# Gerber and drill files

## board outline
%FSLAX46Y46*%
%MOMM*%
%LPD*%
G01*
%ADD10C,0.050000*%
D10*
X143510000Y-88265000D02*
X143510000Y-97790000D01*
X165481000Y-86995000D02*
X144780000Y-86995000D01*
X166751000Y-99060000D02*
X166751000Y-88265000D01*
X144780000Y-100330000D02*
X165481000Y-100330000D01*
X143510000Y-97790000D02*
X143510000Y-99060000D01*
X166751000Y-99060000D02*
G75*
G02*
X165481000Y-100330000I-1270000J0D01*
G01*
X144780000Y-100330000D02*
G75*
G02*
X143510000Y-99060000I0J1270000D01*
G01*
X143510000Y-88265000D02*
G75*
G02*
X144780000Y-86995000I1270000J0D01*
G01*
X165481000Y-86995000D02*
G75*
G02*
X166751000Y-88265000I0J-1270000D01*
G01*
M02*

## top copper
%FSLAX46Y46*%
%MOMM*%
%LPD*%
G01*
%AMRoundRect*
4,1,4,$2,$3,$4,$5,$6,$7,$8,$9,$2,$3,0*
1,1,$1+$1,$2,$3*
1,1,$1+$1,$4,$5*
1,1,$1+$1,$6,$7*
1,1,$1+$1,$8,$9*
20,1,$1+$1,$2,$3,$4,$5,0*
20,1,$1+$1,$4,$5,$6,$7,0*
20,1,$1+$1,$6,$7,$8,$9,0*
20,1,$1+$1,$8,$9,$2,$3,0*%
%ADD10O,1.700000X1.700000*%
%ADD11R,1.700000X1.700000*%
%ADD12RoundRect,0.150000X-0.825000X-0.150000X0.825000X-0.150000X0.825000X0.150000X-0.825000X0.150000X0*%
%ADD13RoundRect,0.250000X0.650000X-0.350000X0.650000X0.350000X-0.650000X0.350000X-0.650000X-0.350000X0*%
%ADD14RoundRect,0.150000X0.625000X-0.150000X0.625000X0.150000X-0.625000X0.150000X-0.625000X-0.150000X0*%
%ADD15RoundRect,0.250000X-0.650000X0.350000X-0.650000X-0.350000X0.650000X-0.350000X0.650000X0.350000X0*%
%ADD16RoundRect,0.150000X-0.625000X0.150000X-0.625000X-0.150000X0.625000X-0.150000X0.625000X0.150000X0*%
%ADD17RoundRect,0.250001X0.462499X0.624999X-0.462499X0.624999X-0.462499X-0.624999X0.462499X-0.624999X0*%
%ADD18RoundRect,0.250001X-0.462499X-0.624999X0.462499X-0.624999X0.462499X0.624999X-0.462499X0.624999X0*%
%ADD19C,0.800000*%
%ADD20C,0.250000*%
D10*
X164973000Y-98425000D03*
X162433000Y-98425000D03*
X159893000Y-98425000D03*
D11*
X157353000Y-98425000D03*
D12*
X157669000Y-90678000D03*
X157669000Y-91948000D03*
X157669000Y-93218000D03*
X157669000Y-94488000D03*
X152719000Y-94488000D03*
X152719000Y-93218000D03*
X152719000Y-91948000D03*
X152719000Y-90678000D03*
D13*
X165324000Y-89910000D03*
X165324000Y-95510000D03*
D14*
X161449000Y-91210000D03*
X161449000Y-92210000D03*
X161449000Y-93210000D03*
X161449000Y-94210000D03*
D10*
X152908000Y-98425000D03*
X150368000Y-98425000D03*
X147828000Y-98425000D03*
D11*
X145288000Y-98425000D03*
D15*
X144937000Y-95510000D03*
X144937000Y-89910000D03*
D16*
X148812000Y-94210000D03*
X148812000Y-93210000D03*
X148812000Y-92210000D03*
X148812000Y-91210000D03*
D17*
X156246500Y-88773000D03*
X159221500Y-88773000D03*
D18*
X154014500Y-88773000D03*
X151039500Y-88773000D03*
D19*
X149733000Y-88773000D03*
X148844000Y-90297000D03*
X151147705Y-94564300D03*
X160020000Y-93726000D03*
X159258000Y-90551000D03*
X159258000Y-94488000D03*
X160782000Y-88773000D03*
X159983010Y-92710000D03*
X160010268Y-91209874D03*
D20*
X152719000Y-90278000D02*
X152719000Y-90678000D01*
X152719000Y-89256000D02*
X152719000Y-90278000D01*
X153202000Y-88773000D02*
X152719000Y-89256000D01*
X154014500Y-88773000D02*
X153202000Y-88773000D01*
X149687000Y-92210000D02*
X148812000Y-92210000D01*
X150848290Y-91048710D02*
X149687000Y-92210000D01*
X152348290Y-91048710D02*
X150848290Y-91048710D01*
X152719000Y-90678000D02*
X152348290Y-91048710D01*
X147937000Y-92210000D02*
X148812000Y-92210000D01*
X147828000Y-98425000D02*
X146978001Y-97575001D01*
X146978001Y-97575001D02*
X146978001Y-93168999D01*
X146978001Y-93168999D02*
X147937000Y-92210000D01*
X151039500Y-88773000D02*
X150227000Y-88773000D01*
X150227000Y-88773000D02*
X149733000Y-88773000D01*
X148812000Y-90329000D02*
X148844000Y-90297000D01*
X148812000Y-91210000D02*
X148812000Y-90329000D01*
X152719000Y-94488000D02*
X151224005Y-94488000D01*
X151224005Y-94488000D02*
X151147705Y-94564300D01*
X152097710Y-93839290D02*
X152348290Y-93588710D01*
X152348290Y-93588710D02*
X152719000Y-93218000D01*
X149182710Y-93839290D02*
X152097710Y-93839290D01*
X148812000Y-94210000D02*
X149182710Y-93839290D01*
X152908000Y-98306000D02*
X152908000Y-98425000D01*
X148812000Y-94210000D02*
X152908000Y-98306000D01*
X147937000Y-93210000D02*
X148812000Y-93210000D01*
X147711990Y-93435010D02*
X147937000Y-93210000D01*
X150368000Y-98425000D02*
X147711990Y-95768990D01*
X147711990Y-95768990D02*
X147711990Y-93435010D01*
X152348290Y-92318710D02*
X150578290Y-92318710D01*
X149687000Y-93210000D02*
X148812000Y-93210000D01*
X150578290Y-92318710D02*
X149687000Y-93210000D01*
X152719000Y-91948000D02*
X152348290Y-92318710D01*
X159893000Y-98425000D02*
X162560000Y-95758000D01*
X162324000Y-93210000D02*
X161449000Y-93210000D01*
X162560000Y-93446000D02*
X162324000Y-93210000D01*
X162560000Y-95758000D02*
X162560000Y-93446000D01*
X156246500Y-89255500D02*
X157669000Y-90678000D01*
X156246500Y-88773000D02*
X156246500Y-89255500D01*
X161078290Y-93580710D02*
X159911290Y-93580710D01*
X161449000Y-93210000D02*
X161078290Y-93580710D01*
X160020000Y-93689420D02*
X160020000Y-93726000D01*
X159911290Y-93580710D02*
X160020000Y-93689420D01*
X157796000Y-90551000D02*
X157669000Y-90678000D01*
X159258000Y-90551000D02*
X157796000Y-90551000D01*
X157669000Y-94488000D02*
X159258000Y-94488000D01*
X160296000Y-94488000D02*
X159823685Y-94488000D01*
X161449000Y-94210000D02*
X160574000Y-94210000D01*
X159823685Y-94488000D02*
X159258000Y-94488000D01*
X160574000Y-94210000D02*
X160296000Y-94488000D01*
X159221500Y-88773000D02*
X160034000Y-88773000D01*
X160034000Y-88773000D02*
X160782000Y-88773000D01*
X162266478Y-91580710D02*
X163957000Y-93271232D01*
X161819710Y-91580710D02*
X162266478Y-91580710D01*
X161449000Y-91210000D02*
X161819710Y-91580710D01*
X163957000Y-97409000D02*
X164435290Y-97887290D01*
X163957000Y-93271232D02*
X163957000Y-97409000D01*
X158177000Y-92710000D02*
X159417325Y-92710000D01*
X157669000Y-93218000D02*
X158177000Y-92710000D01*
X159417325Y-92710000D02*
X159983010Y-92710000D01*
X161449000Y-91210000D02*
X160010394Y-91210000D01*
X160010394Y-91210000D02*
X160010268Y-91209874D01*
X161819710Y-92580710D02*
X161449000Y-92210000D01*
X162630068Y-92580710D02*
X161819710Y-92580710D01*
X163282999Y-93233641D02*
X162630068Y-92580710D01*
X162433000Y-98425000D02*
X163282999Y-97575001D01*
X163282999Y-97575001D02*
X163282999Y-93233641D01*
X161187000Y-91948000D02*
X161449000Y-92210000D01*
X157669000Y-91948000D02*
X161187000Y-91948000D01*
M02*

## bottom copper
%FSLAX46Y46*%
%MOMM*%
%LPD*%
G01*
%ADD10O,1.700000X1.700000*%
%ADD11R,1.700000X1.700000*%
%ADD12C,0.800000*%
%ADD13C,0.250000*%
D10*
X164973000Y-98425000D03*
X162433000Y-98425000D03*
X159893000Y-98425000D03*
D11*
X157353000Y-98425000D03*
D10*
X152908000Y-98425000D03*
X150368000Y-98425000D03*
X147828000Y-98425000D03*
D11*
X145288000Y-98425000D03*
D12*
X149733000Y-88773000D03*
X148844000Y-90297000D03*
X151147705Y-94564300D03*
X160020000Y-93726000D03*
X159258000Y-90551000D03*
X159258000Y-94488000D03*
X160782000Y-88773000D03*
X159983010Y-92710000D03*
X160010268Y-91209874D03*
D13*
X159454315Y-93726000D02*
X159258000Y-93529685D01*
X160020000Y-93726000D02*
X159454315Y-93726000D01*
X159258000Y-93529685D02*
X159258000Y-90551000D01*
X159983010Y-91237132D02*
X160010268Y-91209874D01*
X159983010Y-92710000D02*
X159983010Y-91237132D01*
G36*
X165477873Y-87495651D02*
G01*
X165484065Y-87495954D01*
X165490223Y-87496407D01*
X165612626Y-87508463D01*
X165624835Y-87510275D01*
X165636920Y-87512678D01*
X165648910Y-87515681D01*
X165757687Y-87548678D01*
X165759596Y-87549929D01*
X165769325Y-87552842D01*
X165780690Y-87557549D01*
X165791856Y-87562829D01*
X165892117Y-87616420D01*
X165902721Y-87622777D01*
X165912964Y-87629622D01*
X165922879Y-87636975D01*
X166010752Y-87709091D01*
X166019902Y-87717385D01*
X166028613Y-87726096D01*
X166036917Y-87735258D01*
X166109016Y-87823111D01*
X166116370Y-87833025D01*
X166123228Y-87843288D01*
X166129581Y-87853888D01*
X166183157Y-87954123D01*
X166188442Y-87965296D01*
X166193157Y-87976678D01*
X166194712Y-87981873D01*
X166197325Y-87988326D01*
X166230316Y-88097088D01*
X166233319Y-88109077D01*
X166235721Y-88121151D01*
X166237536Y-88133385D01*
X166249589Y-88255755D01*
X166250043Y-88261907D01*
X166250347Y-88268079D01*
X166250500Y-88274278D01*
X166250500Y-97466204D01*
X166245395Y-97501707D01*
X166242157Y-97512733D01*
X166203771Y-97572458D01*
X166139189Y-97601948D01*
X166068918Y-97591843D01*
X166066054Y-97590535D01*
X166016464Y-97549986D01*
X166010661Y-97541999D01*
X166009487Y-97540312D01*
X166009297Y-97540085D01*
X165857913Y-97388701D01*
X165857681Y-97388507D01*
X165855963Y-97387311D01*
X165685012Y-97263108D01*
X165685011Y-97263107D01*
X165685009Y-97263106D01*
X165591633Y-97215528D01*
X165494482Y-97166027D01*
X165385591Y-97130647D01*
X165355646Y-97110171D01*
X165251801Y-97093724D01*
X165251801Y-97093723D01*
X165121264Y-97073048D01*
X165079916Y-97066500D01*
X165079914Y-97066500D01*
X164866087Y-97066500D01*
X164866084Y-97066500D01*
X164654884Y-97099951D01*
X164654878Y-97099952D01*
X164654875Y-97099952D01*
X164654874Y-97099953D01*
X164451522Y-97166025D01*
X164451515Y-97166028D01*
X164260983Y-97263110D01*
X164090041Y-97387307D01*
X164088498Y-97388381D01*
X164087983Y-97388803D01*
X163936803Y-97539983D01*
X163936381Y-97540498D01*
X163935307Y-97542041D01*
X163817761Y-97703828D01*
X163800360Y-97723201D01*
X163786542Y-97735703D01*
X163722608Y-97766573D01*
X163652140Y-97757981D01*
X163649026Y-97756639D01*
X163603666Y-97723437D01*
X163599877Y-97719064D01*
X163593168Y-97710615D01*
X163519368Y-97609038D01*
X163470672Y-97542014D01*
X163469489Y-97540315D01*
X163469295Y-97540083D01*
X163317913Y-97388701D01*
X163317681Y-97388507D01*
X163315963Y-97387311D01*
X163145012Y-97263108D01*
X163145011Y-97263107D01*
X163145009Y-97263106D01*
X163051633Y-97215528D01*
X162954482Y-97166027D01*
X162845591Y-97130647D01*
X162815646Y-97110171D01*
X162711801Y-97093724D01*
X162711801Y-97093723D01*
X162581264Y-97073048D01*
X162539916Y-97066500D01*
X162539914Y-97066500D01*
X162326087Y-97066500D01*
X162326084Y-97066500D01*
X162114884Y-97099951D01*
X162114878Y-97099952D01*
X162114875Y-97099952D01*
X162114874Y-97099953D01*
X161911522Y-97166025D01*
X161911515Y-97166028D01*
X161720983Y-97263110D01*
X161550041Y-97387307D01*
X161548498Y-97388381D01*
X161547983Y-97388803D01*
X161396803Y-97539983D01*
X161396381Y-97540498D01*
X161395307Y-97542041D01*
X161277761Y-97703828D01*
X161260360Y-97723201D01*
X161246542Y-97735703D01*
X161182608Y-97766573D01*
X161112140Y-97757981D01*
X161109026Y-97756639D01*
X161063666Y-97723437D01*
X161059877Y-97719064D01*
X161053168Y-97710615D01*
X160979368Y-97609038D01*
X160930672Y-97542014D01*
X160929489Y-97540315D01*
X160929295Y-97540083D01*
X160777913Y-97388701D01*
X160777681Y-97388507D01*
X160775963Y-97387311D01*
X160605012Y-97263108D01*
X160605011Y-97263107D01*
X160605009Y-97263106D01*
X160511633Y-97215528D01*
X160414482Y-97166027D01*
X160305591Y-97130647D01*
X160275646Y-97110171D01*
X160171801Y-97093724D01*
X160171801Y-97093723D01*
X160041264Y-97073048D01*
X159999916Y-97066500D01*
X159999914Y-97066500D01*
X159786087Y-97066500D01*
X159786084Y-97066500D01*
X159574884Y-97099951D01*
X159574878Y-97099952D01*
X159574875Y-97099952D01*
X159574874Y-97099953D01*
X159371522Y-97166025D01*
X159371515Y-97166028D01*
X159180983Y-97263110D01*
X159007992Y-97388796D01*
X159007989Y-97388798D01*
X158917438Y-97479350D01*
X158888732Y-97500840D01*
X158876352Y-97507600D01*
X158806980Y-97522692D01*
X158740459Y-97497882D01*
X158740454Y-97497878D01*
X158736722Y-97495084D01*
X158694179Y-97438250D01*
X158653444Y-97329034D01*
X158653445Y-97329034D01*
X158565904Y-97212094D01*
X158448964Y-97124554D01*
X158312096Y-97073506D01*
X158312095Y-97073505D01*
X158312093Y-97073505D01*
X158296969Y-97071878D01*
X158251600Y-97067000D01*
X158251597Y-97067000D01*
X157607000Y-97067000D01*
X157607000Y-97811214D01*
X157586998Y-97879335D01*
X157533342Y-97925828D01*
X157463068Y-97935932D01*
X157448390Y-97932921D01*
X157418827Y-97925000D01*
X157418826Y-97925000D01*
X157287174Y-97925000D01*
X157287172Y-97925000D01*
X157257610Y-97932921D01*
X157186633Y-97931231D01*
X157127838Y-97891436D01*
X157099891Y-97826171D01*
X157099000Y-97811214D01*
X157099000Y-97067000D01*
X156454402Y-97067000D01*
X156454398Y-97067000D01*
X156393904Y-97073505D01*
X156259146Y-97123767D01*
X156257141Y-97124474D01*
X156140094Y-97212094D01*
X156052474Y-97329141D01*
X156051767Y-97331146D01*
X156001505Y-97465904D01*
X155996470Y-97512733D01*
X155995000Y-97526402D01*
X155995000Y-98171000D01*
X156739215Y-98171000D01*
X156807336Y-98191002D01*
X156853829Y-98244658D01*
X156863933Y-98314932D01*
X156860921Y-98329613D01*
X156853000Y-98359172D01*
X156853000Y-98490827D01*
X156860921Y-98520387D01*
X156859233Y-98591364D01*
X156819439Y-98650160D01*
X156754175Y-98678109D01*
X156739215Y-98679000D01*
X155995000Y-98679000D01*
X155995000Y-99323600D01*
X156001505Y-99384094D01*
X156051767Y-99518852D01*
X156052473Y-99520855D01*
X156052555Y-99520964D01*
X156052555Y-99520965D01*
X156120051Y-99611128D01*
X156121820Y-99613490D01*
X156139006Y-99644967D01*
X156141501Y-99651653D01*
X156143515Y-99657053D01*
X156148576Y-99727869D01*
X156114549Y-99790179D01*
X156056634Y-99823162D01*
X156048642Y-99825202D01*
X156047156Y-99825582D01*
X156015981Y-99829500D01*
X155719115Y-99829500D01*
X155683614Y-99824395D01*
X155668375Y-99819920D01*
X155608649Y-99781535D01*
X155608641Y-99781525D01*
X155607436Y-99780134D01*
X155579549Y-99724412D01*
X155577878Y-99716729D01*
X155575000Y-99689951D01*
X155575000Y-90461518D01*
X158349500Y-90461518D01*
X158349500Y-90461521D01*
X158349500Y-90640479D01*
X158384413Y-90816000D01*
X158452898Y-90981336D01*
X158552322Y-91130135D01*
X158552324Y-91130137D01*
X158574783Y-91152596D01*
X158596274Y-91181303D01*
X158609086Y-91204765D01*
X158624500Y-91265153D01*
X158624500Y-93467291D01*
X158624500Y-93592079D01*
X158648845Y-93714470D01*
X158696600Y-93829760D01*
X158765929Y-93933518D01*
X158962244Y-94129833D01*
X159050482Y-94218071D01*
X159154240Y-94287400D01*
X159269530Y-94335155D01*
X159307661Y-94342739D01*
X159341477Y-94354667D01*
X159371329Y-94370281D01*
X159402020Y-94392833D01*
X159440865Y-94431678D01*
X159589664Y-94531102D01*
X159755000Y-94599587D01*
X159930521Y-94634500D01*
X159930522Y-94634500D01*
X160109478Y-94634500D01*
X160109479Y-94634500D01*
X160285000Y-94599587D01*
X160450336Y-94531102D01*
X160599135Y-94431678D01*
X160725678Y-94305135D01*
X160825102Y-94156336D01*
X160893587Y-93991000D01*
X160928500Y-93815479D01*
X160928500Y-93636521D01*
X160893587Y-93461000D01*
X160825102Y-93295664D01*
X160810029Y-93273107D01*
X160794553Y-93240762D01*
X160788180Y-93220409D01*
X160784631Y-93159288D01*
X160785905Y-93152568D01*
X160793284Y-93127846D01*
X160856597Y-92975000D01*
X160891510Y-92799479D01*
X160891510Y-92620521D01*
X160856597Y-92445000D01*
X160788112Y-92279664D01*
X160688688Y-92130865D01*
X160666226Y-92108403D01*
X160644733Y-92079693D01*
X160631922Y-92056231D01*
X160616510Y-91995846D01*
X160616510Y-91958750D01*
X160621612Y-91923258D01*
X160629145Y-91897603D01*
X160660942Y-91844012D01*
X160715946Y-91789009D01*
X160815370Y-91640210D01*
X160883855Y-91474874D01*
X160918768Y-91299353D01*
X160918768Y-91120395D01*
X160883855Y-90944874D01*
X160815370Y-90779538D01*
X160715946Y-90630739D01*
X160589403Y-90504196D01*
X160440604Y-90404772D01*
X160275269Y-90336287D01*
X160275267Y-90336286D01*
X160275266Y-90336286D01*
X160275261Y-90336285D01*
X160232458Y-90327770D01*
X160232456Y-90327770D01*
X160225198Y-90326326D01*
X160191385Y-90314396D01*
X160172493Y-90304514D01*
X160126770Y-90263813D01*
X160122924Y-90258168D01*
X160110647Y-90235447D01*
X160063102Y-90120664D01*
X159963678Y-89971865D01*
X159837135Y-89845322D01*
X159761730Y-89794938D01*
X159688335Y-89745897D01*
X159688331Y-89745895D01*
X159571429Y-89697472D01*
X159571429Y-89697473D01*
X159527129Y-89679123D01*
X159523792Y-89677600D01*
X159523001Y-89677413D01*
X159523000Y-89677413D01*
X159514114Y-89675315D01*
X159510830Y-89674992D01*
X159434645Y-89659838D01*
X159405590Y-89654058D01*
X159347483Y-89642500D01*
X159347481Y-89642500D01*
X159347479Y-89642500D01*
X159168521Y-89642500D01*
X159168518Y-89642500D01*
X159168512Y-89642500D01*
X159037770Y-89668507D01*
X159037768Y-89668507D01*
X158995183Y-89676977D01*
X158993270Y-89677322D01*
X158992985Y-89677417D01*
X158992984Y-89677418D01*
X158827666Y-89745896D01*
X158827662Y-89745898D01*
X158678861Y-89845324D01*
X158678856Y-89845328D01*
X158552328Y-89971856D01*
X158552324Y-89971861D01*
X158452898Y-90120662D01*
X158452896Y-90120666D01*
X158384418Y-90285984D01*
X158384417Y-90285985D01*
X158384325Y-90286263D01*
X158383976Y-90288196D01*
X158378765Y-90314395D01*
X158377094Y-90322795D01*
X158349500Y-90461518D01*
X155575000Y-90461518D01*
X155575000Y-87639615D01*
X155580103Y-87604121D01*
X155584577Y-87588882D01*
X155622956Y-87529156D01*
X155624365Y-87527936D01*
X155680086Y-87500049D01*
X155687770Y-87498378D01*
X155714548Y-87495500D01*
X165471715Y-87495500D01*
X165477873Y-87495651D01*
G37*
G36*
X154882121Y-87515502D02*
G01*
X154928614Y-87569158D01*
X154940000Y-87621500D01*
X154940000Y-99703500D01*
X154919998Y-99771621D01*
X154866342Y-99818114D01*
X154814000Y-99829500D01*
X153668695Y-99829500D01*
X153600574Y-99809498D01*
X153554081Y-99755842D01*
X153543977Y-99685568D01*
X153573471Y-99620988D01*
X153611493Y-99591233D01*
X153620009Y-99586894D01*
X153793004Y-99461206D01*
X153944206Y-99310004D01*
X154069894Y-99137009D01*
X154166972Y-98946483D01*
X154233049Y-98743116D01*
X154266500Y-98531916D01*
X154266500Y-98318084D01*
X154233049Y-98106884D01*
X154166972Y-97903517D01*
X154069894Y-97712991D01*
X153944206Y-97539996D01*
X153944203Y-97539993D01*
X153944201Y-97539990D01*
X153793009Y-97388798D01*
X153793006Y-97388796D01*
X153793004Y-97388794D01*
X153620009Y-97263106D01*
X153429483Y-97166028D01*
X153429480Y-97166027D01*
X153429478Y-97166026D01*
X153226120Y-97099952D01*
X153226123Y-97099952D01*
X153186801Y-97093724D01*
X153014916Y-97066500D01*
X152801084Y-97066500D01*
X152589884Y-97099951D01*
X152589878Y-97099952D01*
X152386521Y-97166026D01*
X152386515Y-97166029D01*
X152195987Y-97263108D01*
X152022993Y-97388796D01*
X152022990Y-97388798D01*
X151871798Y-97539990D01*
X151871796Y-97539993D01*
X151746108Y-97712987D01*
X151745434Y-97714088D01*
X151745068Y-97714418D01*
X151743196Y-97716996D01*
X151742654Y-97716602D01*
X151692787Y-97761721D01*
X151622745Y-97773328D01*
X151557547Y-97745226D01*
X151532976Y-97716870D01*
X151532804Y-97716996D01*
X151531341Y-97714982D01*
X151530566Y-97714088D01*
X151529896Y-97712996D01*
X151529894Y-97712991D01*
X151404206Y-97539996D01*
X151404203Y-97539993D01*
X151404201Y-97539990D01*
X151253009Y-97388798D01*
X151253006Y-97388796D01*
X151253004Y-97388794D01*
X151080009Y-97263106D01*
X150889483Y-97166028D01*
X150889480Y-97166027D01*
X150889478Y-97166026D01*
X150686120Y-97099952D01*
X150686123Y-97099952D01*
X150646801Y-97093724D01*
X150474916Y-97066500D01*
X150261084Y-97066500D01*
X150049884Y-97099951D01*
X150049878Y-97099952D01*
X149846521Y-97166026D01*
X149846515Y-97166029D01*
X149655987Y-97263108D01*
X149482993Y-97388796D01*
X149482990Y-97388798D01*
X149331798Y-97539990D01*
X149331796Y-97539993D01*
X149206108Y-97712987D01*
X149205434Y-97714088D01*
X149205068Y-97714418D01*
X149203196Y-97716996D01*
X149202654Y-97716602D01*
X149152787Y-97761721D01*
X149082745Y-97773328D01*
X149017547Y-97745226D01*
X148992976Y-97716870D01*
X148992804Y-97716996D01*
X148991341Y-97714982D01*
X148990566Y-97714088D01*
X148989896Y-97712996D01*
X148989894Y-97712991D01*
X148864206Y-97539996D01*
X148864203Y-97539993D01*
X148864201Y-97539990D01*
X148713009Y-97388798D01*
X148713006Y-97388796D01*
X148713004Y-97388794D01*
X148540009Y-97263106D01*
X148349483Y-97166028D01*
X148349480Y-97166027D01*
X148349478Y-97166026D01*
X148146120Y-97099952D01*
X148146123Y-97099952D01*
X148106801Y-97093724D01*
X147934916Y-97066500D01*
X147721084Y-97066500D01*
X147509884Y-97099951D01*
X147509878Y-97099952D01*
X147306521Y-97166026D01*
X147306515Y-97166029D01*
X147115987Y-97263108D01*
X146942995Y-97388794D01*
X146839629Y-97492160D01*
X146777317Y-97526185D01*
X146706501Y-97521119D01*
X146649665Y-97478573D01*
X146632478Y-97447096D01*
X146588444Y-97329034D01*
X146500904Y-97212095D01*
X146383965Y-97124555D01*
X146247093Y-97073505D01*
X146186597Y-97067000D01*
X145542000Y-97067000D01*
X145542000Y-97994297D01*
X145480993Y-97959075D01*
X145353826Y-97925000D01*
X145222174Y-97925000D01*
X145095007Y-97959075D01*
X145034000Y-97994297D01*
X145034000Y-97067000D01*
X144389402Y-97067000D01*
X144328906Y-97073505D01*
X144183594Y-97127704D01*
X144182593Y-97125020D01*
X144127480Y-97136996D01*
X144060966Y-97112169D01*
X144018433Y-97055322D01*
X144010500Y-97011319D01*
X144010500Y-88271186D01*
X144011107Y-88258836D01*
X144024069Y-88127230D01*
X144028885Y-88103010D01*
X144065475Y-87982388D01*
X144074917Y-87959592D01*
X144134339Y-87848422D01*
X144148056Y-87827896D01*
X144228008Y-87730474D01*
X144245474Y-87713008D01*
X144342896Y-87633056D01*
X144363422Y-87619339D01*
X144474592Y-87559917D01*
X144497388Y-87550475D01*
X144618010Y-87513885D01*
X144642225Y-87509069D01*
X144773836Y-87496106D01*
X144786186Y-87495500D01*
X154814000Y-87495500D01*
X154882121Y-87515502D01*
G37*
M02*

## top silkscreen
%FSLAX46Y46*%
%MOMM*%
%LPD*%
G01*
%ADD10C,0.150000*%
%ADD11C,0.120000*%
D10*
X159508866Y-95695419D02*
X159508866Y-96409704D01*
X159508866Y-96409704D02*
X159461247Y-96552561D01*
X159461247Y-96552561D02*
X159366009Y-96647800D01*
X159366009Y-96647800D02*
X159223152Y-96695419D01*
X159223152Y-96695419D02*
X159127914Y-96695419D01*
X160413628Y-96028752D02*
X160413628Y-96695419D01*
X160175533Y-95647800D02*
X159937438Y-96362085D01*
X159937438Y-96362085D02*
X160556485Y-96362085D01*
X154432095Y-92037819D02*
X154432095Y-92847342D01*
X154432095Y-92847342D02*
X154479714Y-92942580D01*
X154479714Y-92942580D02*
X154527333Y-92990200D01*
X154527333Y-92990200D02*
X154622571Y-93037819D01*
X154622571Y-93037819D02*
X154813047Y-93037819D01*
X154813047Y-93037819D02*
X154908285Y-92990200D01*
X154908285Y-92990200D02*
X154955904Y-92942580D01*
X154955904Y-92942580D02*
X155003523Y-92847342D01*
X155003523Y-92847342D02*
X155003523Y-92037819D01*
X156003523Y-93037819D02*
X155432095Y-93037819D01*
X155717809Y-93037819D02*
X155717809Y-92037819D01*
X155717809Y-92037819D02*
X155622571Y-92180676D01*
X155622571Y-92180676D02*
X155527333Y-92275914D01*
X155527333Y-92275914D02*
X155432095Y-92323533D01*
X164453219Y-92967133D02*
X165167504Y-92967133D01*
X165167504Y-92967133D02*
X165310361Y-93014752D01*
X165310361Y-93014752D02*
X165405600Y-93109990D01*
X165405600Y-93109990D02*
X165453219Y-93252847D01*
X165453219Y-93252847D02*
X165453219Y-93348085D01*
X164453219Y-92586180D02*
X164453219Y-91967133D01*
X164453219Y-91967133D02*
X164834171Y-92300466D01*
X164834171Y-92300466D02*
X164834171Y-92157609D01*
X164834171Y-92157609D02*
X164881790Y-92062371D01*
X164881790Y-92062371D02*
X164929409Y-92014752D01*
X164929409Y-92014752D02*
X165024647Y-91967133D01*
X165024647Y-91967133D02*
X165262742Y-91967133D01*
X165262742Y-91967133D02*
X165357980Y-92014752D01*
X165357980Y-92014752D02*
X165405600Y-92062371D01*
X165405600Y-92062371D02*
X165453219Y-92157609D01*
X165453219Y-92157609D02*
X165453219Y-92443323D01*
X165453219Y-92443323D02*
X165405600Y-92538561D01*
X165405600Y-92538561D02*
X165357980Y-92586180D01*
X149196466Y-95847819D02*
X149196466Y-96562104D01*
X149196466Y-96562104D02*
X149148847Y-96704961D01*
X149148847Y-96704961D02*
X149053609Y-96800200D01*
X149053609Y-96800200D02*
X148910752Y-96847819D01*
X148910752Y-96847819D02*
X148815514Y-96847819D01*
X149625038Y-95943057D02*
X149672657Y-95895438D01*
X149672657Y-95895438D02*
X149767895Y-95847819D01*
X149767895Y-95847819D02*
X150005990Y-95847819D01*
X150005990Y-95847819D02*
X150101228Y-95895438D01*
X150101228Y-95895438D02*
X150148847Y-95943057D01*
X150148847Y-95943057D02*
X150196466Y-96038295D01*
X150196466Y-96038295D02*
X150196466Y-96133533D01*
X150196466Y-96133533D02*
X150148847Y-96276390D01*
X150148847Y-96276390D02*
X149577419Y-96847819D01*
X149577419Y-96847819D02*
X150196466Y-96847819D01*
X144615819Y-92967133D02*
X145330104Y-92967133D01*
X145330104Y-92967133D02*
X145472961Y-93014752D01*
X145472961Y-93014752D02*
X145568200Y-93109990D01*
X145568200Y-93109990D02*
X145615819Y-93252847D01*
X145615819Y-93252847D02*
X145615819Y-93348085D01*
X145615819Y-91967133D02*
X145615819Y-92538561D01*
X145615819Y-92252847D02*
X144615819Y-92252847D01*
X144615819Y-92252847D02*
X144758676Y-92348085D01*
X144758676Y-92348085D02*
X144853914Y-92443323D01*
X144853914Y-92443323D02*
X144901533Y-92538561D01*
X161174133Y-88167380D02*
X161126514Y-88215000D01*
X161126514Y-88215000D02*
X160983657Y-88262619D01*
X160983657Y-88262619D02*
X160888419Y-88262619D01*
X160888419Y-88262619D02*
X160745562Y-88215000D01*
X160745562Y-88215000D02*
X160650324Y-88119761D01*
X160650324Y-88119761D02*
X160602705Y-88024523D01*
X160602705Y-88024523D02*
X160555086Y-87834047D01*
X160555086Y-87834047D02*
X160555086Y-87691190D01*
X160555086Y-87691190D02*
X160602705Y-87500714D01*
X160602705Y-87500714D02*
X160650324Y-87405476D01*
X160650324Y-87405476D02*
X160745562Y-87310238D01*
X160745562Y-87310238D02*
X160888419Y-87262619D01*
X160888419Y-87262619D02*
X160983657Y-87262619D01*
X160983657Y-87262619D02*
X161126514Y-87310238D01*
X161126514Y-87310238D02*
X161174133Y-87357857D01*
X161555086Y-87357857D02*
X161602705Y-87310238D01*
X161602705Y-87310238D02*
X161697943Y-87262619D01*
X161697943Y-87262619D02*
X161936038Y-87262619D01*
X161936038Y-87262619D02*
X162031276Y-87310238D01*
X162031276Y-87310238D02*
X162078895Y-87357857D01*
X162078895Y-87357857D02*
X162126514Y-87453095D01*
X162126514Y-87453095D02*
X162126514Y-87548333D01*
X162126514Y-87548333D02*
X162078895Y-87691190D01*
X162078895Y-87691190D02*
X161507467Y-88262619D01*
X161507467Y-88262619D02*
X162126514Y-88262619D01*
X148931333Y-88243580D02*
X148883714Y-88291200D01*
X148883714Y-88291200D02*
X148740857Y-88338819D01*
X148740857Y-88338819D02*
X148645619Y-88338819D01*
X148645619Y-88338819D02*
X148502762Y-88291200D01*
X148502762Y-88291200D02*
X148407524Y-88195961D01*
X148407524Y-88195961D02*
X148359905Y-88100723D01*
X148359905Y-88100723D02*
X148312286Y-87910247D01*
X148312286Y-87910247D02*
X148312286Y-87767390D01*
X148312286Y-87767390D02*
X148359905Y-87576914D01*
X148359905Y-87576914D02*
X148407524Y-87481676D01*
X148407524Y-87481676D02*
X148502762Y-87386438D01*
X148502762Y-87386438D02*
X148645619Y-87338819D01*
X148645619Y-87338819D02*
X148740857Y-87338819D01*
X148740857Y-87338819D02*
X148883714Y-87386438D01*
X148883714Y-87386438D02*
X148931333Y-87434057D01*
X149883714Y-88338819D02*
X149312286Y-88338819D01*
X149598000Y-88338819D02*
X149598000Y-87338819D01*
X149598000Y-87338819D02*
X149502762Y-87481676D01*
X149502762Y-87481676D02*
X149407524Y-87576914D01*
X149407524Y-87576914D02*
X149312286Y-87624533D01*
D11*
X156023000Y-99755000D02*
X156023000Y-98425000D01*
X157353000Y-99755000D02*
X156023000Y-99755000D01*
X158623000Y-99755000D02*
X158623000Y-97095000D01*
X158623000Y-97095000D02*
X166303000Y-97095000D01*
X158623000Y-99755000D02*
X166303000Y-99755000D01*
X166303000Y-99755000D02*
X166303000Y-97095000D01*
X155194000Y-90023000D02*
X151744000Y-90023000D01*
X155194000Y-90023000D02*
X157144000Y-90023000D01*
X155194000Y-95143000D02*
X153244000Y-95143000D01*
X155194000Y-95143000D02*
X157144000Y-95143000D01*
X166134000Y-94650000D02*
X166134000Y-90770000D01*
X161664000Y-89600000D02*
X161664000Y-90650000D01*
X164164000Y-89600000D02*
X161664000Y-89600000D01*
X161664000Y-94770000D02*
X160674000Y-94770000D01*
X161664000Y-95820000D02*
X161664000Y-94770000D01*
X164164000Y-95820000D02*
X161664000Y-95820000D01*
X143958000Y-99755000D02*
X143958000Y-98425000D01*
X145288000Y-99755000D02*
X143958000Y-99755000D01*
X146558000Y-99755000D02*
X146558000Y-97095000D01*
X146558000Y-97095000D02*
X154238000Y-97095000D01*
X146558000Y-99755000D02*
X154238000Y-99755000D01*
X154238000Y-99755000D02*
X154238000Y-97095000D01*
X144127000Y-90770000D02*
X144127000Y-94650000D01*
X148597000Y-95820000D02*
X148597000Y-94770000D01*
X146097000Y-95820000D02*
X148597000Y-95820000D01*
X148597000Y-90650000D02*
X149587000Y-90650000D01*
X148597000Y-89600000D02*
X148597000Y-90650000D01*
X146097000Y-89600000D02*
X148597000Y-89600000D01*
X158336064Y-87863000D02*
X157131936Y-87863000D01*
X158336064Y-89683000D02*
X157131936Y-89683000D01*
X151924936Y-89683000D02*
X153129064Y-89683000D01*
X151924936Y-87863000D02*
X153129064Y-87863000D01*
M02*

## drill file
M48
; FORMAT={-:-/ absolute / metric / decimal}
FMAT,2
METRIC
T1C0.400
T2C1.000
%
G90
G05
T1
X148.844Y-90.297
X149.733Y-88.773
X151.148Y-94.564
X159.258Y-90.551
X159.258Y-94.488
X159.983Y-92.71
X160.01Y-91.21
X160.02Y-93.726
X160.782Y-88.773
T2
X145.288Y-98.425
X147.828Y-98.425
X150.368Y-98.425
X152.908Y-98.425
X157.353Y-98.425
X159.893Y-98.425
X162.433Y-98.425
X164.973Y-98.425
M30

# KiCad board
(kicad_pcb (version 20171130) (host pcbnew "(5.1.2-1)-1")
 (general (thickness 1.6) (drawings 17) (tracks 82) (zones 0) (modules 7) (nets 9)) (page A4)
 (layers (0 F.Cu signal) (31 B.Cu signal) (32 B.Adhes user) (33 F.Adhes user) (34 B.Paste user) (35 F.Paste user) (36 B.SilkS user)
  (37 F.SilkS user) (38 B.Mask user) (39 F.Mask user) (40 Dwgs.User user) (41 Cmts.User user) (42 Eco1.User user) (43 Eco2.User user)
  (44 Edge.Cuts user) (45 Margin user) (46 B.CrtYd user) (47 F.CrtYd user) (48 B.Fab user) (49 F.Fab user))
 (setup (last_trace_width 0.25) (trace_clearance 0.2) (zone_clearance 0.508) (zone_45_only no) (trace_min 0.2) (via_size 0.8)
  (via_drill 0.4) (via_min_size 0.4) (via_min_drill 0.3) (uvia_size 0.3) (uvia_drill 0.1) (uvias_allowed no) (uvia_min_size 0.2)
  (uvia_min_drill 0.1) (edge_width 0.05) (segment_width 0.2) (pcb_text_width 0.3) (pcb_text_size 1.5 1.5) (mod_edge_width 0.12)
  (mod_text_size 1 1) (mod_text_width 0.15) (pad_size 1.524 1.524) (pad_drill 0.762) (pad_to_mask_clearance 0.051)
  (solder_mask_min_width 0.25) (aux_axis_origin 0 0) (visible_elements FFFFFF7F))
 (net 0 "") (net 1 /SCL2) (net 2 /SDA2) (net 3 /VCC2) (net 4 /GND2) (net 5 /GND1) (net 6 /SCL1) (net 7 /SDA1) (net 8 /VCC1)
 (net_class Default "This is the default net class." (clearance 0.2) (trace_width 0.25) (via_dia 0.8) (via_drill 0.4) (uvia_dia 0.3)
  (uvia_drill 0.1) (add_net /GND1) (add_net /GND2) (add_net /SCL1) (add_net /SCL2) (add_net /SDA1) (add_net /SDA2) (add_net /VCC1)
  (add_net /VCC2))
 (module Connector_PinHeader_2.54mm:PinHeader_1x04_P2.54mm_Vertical (layer F.Cu) (at 157.353 98.425 90)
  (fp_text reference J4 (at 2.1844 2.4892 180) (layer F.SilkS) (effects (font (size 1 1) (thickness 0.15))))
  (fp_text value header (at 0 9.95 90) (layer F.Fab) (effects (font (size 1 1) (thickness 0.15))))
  (fp_line (start -1.33 -1.33) (end 0 -1.33) (layer F.SilkS) (width 0.12))
  (fp_line (start -1.33 0) (end -1.33 -1.33) (layer F.SilkS) (width 0.12))
  (fp_line (start -1.33 1.27) (end 1.33 1.27) (layer F.SilkS) (width 0.12))
  (fp_line (start 1.33 1.27) (end 1.33 8.95) (layer F.SilkS) (width 0.12))
  (fp_line (start -1.33 1.27) (end -1.33 8.95) (layer F.SilkS) (width 0.12))
  (fp_line (start -1.33 8.95) (end 1.33 8.95) (layer F.SilkS) (width 0.12))
  (pad 4 thru_hole oval (at 0 7.62 90) (size 1.7 1.7) (drill 1) (layers *.Cu *.Mask) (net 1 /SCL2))
  (pad 3 thru_hole oval (at 0 5.08 90) (size 1.7 1.7) (drill 1) (layers *.Cu *.Mask) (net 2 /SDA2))
  (pad 2 thru_hole oval (at 0 2.54 90) (size 1.7 1.7) (drill 1) (layers *.Cu *.Mask) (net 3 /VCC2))
  (pad 1 thru_hole rect (at 0 0 90) (size 1.7 1.7) (drill 1) (layers *.Cu *.Mask) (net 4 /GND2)))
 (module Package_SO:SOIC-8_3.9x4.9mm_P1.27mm (layer F.Cu) (at 155.194 92.583)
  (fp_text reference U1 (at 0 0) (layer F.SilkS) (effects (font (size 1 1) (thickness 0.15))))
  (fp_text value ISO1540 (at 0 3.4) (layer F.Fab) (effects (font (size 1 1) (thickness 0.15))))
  (fp_line (start 0 -2.56) (end -3.45 -2.56) (layer F.SilkS) (width 0.12))
  (fp_line (start 0 -2.56) (end 1.95 -2.56) (layer F.SilkS) (width 0.12))
  (fp_line (start 0 2.56) (end -1.95 2.56) (layer F.SilkS) (width 0.12))
  (fp_line (start 0 2.56) (end 1.95 2.56) (layer F.SilkS) (width 0.12))
  (pad 8 smd roundrect (at 2.475 -1.905) (size 1.95 0.6) (layers F.Cu F.Paste F.Mask) (roundrect_rratio 0.25) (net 3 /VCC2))
  (pad 7 smd roundrect (at 2.475 -0.635) (size 1.95 0.6) (layers F.Cu F.Paste F.Mask) (roundrect_rratio 0.25) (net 2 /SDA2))
  (pad 6 smd roundrect (at 2.475 0.635) (size 1.95 0.6) (layers F.Cu F.Paste F.Mask) (roundrect_rratio 0.25) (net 1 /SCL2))
  (pad 5 smd roundrect (at 2.475 1.905) (size 1.95 0.6) (layers F.Cu F.Paste F.Mask) (roundrect_rratio 0.25) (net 4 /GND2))
  (pad 4 smd roundrect (at -2.475 1.905) (size 1.95 0.6) (layers F.Cu F.Paste F.Mask) (roundrect_rratio 0.25) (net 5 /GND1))
  (pad 3 smd roundrect (at -2.475 0.635) (size 1.95 0.6) (layers F.Cu F.Paste F.Mask) (roundrect_rratio 0.25) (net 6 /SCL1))
  (pad 2 smd roundrect (at -2.475 -0.635) (size 1.95 0.6) (layers F.Cu F.Paste F.Mask) (roundrect_rratio 0.25) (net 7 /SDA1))
  (pad 1 smd roundrect (at -2.475 -1.905) (size 1.95 0.6) (layers F.Cu F.Paste F.Mask) (roundrect_rratio 0.25) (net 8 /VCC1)))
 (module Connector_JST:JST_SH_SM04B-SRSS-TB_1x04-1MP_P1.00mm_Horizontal (layer F.Cu) (at 163.449 92.71 90)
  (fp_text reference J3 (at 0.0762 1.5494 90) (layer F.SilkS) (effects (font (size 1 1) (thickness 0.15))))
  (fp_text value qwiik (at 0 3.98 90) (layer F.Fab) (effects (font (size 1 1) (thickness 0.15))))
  (fp_line (start -1.94 2.685) (end 1.94 2.685) (layer F.SilkS) (width 0.12))
  (fp_line (start 3.11 -1.785) (end 2.06 -1.785) (layer F.SilkS) (width 0.12))
  (fp_line (start 3.11 0.715) (end 3.11 -1.785) (layer F.SilkS) (width 0.12))
  (fp_line (start -2.06 -1.785) (end -2.06 -2.775) (layer F.SilkS) (width 0.12))
  (fp_line (start -3.11 -1.785) (end -2.06 -1.785) (layer F.SilkS) (width 0.12))
  (fp_line (start -3.11 0.715) (end -3.11 -1.785) (layer F.SilkS) (width 0.12))
  (pad MP smd roundrect (at 2.8 1.875 90) (size 1.2 1.8) (layers F.Cu F.Paste F.Mask) (roundrect_rratio 0.208333))
  (pad MP smd roundrect (at -2.8 1.875 90) (size 1.2 1.8) (layers F.Cu F.Paste F.Mask) (roundrect_rratio 0.208333))
  (pad 4 smd roundrect (at 1.5 -2 90) (size 0.6 1.55) (layers F.Cu F.Paste F.Mask) (roundrect_rratio 0.25) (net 1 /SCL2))
  (pad 3 smd roundrect (at 0.5 -2 90) (size 0.6 1.55) (layers F.Cu F.Paste F.Mask) (roundrect_rratio 0.25) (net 2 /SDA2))
  (pad 2 smd roundrect (at -0.5 -2 90) (size 0.6 1.55) (layers F.Cu F.Paste F.Mask) (roundrect_rratio 0.25) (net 3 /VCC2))
  (pad 1 smd roundrect (at -1.5 -2 90) (size 0.6 1.55) (layers F.Cu F.Paste F.Mask) (roundrect_rratio 0.25) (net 4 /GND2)))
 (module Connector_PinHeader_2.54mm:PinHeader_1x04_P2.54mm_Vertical (layer F.Cu) (at 145.288 98.425 90)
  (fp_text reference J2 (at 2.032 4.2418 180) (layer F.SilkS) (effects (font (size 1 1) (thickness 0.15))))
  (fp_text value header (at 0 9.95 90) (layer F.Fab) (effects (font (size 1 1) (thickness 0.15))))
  (fp_line (start -1.33 -1.33) (end 0 -1.33) (layer F.SilkS) (width 0.12))
  (fp_line (start -1.33 0) (end -1.33 -1.33) (layer F.SilkS) (width 0.12))
  (fp_line (start -1.33 1.27) (end 1.33 1.27) (layer F.SilkS) (width 0.12))
  (fp_line (start 1.33 1.27) (end 1.33 8.95) (layer F.SilkS) (width 0.12))
  (fp_line (start -1.33 1.27) (end -1.33 8.95) (layer F.SilkS) (width 0.12))
  (fp_line (start -1.33 8.95) (end 1.33 8.95) (layer F.SilkS) (width 0.12))
  (pad 4 thru_hole oval (at 0 7.62 90) (size 1.7 1.7) (drill 1) (layers *.Cu *.Mask) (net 6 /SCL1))
  (pad 3 thru_hole oval (at 0 5.08 90) (size 1.7 1.7) (drill 1) (layers *.Cu *.Mask) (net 7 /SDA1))
  (pad 2 thru_hole oval (at 0 2.54 90) (size 1.7 1.7) (drill 1) (layers *.Cu *.Mask) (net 8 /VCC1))
  (pad 1 thru_hole rect (at 0 0 90) (size 1.7 1.7) (drill 1) (layers *.Cu *.Mask) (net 5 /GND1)))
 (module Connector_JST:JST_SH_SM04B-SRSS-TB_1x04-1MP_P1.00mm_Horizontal (layer F.Cu) (at 146.812 92.71 270)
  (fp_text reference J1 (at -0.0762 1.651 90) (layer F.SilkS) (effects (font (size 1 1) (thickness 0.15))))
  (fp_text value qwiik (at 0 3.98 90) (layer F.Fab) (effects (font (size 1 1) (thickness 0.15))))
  (fp_line (start -1.94 2.685) (end 1.94 2.685) (layer F.SilkS) (width 0.12))
  (fp_line (start 3.11 -1.785) (end 2.06 -1.785) (layer F.SilkS) (width 0.12))
  (fp_line (start 3.11 0.715) (end 3.11 -1.785) (layer F.SilkS) (width 0.12))
  (fp_line (start -2.06 -1.785) (end -2.06 -2.775) (layer F.SilkS) (width 0.12))
  (fp_line (start -3.11 -1.785) (end -2.06 -1.785) (layer F.SilkS) (width 0.12))
  (fp_line (start -3.11 0.715) (end -3.11 -1.785) (layer F.SilkS) (width 0.12))
  (pad MP smd roundrect (at 2.8 1.875 270) (size 1.2 1.8) (layers F.Cu F.Paste F.Mask) (roundrect_rratio 0.208333))
  (pad MP smd roundrect (at -2.8 1.875 270) (size 1.2 1.8) (layers F.Cu F.Paste F.Mask) (roundrect_rratio 0.208333))
  (pad 4 smd roundrect (at 1.5 -2 270) (size 0.6 1.55) (layers F.Cu F.Paste F.Mask) (roundrect_rratio 0.25) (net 6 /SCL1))
  (pad 3 smd roundrect (at 0.5 -2 270) (size 0.6 1.55) (layers F.Cu F.Paste F.Mask) (roundrect_rratio 0.25) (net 7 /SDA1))
  (pad 2 smd roundrect (at -0.5 -2 270) (size 0.6 1.55) (layers F.Cu F.Paste F.Mask) (roundrect_rratio 0.25) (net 8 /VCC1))
  (pad 1 smd roundrect (at -1.5 -2 270) (size 0.6 1.55) (layers F.Cu F.Paste F.Mask) (roundrect_rratio 0.25) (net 5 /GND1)))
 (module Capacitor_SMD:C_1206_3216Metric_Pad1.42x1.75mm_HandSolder (layer F.Cu) (at 157.734 88.773 180)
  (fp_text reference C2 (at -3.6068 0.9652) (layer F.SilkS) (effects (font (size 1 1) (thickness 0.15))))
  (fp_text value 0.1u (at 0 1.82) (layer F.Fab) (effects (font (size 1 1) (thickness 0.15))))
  (fp_line (start -0.602064 0.91) (end 0.602064 0.91) (layer F.SilkS) (width 0.12))
  (fp_line (start -0.602064 -0.91) (end 0.602064 -0.91) (layer F.SilkS) (width 0.12))
  (pad 2 smd roundrect (at 1.4875 0 180) (size 1.425 1.75) (layers F.Cu F.Paste F.Mask) (roundrect_rratio 0.175439) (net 3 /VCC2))
  (pad 1 smd roundrect (at -1.4875 0 180) (size 1.425 1.75) (layers F.Cu F.Paste F.Mask) (roundrect_rratio 0.175439) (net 4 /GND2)))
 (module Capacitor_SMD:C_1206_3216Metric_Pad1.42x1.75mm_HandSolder (layer F.Cu) (at 152.527 88.773)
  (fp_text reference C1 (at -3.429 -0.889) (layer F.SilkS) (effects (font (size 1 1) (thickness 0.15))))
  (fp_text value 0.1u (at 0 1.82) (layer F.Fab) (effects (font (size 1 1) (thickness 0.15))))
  (fp_line (start -0.602064 0.91) (end 0.602064 0.91) (layer F.SilkS) (width 0.12))
  (fp_line (start -0.602064 -0.91) (end 0.602064 -0.91) (layer F.SilkS) (width 0.12))
  (pad 2 smd roundrect (at 1.4875 0) (size 1.425 1.75) (layers F.Cu F.Paste F.Mask) (roundrect_rratio 0.175439) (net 8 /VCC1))
  (pad 1 smd roundrect (at -1.4875 0) (size 1.425 1.75) (layers F.Cu F.Paste F.Mask) (roundrect_rratio 0.175439) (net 5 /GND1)))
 (gr_line (start 143.51 88.265) (end 143.51 97.79) (layer Edge.Cuts) (width 0.05))
 (gr_line (start 165.481 86.995) (end 144.78 86.995) (layer Edge.Cuts) (width 0.05))
 (gr_line (start 166.751 99.06) (end 166.751 88.265) (layer Edge.Cuts) (width 0.05))
 (gr_line (start 144.78 100.33) (end 165.481 100.33) (layer Edge.Cuts) (width 0.05))
 (gr_line (start 143.51 97.79) (end 143.51 99.06) (layer Edge.Cuts) (width 0.05))
 (gr_arc (start 165.481 99.06) (end 165.481 100.33) (angle -90) (layer Edge.Cuts) (width 0.05))
 (gr_arc (start 144.78 99.06) (end 143.51 99.06) (angle -90) (layer Edge.Cuts) (width 0.05))
 (gr_arc (start 144.78 88.265) (end 144.78 86.995) (angle -90) (layer Edge.Cuts) (width 0.05))
 (gr_arc (start 165.481 88.265) (end 166.751 88.265) (angle -90) (layer Edge.Cuts) (width 0.05))
 (segment (start 152.719 90.278) (end 152.719 90.678) (width 0.25) (layer F.Cu) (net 8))
 (segment (start 152.719 89.256) (end 152.719 90.278) (width 0.25) (layer F.Cu) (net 8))
 (segment (start 153.202 88.773) (end 152.719 89.256) (width 0.25) (layer F.Cu) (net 8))
 (segment (start 154.0145 88.773) (end 153.202 88.773) (width 0.25) (layer F.Cu) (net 8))
 (segment (start 149.687 92.21) (end 148.812 92.21) (width 0.25) (layer F.Cu) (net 8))
 (segment (start 150.84829 91.04871) (end 149.687 92.21) (width 0.25) (layer F.Cu) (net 8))
 (segment (start 152.34829 91.04871) (end 150.84829 91.04871) (width 0.25) (layer F.Cu) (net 8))
 (segment (start 152.719 90.678) (end 152.34829 91.04871) (width 0.25) (layer F.Cu) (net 8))
 (segment (start 147.937 92.21) (end 148.812 92.21) (width 0.25) (layer F.Cu) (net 8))
 (segment (start 147.828 98.425) (end 146.978001 97.575001) (width 0.25) (layer F.Cu) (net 8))
 (segment (start 146.978001 97.575001) (end 146.978001 93.168999) (width 0.25) (layer F.Cu) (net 8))
 (segment (start 146.978001 93.168999) (end 147.937 92.21) (width 0.25) (layer F.Cu) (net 8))
 (segment (start 151.0395 88.773) (end 150.227 88.773) (width 0.25) (layer F.Cu) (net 5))
 (via (at 149.733 88.773) (size 0.8) (drill 0.4) (layers F.Cu B.Cu) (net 5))
 (segment (start 150.227 88.773) (end 149.733 88.773) (width 0.25) (layer F.Cu) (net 5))
 (via (at 148.844 90.297) (size 0.8) (drill 0.4) (layers F.Cu B.Cu) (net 5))
 (segment (start 148.812 90.329) (end 148.844 90.297) (width 0.25) (layer F.Cu) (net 5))
 (segment (start 148.812 91.21) (end 148.812 90.329) (width 0.25) (layer F.Cu) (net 5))
 (via (at 151.147705 94.5643) (size 0.8) (drill 0.4) (layers F.Cu B.Cu) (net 5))
 (segment (start 152.719 94.488) (end 151.224005 94.488) (width 0.25) (layer F.Cu) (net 5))
 (segment (start 151.224005 94.488) (end 151.147705 94.5643) (width 0.25) (layer F.Cu) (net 5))
 (segment (start 152.09771 93.83929) (end 152.34829 93.58871) (width 0.25) (layer F.Cu) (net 6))
 (segment (start 152.34829 93.58871) (end 152.719 93.218) (width 0.25) (layer F.Cu) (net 6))
 (segment (start 149.18271 93.83929) (end 152.09771 93.83929) (width 0.25) (layer F.Cu) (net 6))
 (segment (start 148.812 94.21) (end 149.18271 93.83929) (width 0.25) (layer F.Cu) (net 6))
 (segment (start 152.908 98.306) (end 152.908 98.425) (width 0.25) (layer F.Cu) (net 6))
 (segment (start 148.812 94.21) (end 152.908 98.306) (width 0.25) (layer F.Cu) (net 6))
 (segment (start 147.937 93.21) (end 148.812 93.21) (width 0.25) (layer F.Cu) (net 7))
 (segment (start 147.71199 93.43501) (end 147.937 93.21) (width 0.25) (layer F.Cu) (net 7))
 (segment (start 150.368 98.425) (end 147.71199 95.76899) (width 0.25) (layer F.Cu) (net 7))
 (segment (start 147.71199 95.76899) (end 147.71199 93.43501) (width 0.25) (layer F.Cu) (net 7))
 (segment (start 152.34829 92.31871) (end 150.57829 92.31871) (width 0.25) (layer F.Cu) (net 7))
 (segment (start 149.687 93.21) (end 148.812 93.21) (width 0.25) (layer F.Cu) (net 7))
 (segment (start 150.57829 92.31871) (end 149.687 93.21) (width 0.25) (layer F.Cu) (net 7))
 (segment (start 152.719 91.948) (end 152.34829 92.31871) (width 0.25) (layer F.Cu) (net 7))
 (segment (start 159.893 98.425) (end 162.56 95.758) (width 0.25) (layer F.Cu) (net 3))
 (segment (start 162.324 93.21) (end 161.449 93.21) (width 0.25) (layer F.Cu) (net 3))
 (segment (start 162.56 93.446) (end 162.324 93.21) (width 0.25) (layer F.Cu) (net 3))
 (segment (start 162.56 95.758) (end 162.56 93.446) (width 0.25) (layer F.Cu) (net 3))
 (segment (start 156.2465 89.2555) (end 157.669 90.678) (width 0.25) (layer F.Cu) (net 3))
 (segment (start 156.2465 88.773) (end 156.2465 89.2555) (width 0.25) (layer F.Cu) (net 3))
 (segment (start 161.07829 93.58071) (end 159.91129 93.58071) (width 0.25) (layer F.Cu) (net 3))
 (segment (start 161.449 93.21) (end 161.07829 93.58071) (width 0.25) (layer F.Cu) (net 3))
 (via (at 160.02 93.726) (size 0.8) (drill 0.4) (layers F.Cu B.Cu) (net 3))
 (segment (start 160.02 93.68942) (end 160.02 93.726) (width 0.25) (layer F.Cu) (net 3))
 (segment (start 159.91129 93.58071) (end 160.02 93.68942) (width 0.25) (layer F.Cu) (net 3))
 (segment (start 159.454315 93.726) (end 159.258 93.529685) (width 0.25) (layer B.Cu) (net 3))
 (segment (start 160.02 93.726) (end 159.454315 93.726) (width 0.25) (layer B.Cu) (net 3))
 (via (at 159.258 90.551) (size 0.8) (drill 0.4) (layers F.Cu B.Cu) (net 3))
 (segment (start 159.258 93.529685) (end 159.258 90.551) (width 0.25) (layer B.Cu) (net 3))
 (segment (start 157.796 90.551) (end 157.669 90.678) (width 0.25) (layer F.Cu) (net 3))
 (segment (start 159.258 90.551) (end 157.796 90.551) (width 0.25) (layer F.Cu) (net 3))
 (segment (start 157.669 94.488) (end 159.258 94.488) (width 0.25) (layer F.Cu) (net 4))
 (via (at 159.258 94.488) (size 0.8) (drill 0.4) (layers F.Cu B.Cu) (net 4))
 (segment (start 160.296 94.488) (end 159.823685 94.488) (width 0.25) (layer F.Cu) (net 4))
 (segment (start 161.449 94.21) (end 160.574 94.21) (width 0.25) (layer F.Cu) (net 4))
 (segment (start 159.823685 94.488) (end 159.258 94.488) (width 0.25) (layer F.Cu) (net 4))
 (segment (start 160.574 94.21) (end 160.296 94.488) (width 0.25) (layer F.Cu) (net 4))
 (segment (start 159.2215 88.773) (end 160.034 88.773) (width 0.25) (layer F.Cu) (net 4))
 (via (at 160.782 88.773) (size 0.8) (drill 0.4) (layers F.Cu B.Cu) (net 4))
 (segment (start 160.034 88.773) (end 160.782 88.773) (width 0.25) (layer F.Cu) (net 4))
 (segment (start 162.266478 91.58071) (end 163.957 93.271232) (width 0.25) (layer F.Cu) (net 1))
 (segment (start 161.81971 91.58071) (end 162.266478 91.58071) (width 0.25) (layer F.Cu) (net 1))
 (segment (start 161.449 91.21) (end 161.81971 91.58071) (width 0.25) (layer F.Cu) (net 1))
 (segment (start 163.957 97.409) (end 164.43529 97.88729) (width 0.25) (layer F.Cu) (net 1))
 (segment (start 163.957 93.271232) (end 163.957 97.409) (width 0.25) (layer F.Cu) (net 1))
 (via (at 159.98301 92.71) (size 0.8) (drill 0.4) (layers F.Cu B.Cu) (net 1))
 (segment (start 158.177 92.71) (end 159.417325 92.71) (width 0.25) (layer F.Cu) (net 1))
 (segment (start 157.669 93.218) (end 158.177 92.71) (width 0.25) (layer F.Cu) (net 1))
 (segment (start 159.417325 92.71) (end 159.98301 92.71) (width 0.25) (layer F.Cu) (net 1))
 (segment (start 161.449 91.21) (end 160.010394 91.21) (width 0.25) (layer F.Cu) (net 1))
 (segment (start 159.98301 91.237132) (end 160.010268 91.209874) (width 0.25) (layer B.Cu) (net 1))
 (segment (start 160.010394 91.21) (end 160.010268 91.209874) (width 0.25) (layer F.Cu) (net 1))
 (via (at 160.010268 91.209874) (size 0.8) (drill 0.4) (layers F.Cu B.Cu) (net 1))
 (segment (start 159.98301 92.71) (end 159.98301 91.237132) (width 0.25) (layer B.Cu) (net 1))
 (segment (start 161.81971 92.58071) (end 161.449 92.21) (width 0.25) (layer F.Cu) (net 2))
 (segment (start 162.630068 92.58071) (end 161.81971 92.58071) (width 0.25) (layer F.Cu) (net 2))
 (segment (start 163.282999 93.233641) (end 162.630068 92.58071) (width 0.25) (layer F.Cu) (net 2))
 (segment (start 162.433 98.425) (end 163.282999 97.575001) (width 0.25) (layer F.Cu) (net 2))
 (segment (start 163.282999 97.575001) (end 163.282999 93.233641) (width 0.25) (layer F.Cu) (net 2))
 (segment (start 161.187 91.948) (end 161.449 92.21) (width 0.25) (layer F.Cu) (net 2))
 (segment (start 157.669 91.948) (end 161.187 91.948) (width 0.25) (layer F.Cu) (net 2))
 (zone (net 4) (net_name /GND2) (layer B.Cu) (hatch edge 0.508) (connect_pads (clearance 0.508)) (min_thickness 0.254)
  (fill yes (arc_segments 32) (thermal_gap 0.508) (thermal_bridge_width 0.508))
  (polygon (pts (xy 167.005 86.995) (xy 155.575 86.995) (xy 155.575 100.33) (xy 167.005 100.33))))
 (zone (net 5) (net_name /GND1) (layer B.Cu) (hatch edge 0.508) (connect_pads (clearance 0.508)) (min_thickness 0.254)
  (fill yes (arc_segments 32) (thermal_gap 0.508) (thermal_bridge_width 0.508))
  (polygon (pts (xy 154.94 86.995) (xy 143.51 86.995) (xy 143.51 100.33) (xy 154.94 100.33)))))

